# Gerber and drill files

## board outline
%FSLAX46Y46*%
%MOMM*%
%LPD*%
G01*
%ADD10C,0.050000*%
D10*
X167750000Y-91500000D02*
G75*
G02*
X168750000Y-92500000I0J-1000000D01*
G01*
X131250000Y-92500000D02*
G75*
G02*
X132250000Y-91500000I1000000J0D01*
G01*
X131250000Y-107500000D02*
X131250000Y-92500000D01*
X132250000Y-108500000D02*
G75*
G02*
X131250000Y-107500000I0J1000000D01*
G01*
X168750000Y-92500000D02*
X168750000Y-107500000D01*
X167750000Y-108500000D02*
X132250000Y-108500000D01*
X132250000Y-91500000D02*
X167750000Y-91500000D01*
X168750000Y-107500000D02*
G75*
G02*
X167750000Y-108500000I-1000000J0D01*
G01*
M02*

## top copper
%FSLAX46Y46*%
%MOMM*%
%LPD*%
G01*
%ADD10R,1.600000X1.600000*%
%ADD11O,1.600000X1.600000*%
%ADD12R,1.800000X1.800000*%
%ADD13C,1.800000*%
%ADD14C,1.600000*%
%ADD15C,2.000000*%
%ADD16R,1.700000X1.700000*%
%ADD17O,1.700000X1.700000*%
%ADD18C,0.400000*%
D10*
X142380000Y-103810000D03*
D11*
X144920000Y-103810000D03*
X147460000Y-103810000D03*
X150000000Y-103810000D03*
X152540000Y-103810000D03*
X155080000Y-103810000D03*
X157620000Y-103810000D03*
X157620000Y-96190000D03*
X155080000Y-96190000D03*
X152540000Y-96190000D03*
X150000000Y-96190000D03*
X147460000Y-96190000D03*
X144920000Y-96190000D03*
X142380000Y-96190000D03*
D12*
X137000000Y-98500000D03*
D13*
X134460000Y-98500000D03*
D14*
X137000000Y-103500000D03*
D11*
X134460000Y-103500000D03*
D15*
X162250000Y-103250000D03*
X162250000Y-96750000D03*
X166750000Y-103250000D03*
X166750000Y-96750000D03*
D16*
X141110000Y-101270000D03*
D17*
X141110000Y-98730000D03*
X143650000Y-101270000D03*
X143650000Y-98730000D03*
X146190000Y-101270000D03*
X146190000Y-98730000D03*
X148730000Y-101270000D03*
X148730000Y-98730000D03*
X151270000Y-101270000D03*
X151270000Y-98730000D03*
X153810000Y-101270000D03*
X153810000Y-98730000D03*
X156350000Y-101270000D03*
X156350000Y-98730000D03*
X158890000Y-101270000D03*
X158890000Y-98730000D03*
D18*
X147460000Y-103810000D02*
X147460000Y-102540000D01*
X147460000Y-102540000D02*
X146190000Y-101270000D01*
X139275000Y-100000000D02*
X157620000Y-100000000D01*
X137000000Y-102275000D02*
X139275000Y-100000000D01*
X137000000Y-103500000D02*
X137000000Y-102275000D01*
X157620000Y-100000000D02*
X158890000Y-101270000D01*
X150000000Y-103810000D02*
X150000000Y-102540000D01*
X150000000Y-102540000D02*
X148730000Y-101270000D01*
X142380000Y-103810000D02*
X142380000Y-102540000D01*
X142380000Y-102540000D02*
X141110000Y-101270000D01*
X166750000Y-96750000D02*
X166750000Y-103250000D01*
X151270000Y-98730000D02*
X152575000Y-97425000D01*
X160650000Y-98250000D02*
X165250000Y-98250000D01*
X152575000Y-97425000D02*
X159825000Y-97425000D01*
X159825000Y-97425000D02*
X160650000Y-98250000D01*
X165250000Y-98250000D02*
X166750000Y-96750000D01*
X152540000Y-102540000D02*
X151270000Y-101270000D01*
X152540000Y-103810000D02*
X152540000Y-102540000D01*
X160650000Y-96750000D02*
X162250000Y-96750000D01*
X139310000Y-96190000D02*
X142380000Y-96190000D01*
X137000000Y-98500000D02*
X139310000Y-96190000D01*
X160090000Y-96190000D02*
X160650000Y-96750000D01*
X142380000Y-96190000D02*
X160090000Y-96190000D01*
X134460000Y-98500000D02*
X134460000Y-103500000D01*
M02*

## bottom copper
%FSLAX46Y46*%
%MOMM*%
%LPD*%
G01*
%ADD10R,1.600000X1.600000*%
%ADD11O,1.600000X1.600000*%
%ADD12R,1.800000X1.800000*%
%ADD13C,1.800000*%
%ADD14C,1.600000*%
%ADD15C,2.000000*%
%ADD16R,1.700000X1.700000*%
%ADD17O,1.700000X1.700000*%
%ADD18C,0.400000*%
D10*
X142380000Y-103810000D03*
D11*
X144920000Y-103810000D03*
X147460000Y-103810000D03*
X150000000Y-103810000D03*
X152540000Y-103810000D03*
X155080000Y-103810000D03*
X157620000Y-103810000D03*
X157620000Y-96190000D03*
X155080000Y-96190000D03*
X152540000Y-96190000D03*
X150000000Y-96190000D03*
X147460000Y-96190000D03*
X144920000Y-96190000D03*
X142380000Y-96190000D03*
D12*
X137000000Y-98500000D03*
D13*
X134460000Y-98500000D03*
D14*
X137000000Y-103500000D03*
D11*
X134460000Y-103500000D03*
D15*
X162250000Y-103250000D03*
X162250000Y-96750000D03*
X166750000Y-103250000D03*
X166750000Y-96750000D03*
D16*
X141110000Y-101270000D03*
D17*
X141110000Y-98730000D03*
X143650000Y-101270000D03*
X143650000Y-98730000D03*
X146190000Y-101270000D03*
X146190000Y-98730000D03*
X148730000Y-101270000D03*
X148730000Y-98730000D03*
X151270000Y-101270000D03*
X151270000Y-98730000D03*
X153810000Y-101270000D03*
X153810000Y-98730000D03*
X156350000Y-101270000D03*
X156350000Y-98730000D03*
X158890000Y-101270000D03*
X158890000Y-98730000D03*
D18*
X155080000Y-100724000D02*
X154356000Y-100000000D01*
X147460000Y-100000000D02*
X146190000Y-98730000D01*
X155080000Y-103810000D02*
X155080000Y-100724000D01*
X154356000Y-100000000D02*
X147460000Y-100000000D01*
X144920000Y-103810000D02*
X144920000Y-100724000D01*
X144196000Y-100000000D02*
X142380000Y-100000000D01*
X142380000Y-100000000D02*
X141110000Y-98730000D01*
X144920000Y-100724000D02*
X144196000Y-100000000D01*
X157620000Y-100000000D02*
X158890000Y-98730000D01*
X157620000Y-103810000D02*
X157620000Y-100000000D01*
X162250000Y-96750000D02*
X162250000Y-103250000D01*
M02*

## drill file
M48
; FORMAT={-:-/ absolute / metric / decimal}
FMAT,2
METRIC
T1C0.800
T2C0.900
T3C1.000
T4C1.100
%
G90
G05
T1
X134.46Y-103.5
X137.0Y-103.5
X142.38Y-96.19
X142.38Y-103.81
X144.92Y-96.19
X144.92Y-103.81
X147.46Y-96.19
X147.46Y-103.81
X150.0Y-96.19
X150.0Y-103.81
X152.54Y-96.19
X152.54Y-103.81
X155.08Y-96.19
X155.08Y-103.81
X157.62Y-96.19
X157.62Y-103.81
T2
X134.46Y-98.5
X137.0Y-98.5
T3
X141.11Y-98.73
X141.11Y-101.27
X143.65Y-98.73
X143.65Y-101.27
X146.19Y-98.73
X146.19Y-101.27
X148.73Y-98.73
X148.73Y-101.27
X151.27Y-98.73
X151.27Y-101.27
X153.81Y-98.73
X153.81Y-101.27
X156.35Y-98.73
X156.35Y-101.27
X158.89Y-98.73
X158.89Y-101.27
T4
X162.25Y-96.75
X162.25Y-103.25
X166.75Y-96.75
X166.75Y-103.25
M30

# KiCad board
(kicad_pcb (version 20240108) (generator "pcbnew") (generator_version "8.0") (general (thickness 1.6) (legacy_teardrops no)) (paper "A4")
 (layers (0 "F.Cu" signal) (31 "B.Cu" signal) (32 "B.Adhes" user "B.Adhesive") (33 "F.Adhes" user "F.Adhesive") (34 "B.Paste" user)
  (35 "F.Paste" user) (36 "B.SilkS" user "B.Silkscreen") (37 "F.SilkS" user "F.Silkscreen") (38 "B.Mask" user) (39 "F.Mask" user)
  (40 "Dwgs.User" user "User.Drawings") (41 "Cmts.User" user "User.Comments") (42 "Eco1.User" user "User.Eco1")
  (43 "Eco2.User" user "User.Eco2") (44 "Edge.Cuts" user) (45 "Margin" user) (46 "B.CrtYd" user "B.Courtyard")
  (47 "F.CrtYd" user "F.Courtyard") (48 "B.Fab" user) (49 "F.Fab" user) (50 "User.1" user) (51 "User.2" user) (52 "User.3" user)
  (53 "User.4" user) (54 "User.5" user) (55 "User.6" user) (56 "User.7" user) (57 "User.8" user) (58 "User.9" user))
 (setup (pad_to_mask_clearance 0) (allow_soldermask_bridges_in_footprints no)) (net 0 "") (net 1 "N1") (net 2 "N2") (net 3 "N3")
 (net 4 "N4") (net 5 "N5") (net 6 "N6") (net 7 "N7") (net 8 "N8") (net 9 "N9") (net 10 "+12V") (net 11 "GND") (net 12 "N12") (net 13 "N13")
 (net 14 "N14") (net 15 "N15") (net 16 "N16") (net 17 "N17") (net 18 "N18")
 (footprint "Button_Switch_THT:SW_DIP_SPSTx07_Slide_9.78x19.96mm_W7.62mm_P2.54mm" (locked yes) (layer "F.Cu") (at 142.38 103.81 90)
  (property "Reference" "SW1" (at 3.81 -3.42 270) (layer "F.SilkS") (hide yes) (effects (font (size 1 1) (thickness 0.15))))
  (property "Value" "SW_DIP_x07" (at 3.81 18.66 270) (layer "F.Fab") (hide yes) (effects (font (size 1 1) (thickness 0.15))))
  (pad "1" thru_hole rect (at 0 0 90) (size 1.6 1.6) (drill 0.8) (layers "*.Cu" "*.Mask") (remove_unused_layers no) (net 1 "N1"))
  (pad "2" thru_hole oval (at 0 2.54 90) (size 1.6 1.6) (drill 0.8) (layers "*.Cu" "*.Mask") (remove_unused_layers no) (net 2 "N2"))
  (pad "3" thru_hole oval (at 0 5.08 90) (size 1.6 1.6) (drill 0.8) (layers "*.Cu" "*.Mask") (remove_unused_layers no) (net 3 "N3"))
  (pad "4" thru_hole oval (at 0 7.62 90) (size 1.6 1.6) (drill 0.8) (layers "*.Cu" "*.Mask") (remove_unused_layers no) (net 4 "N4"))
  (pad "5" thru_hole oval (at 0 10.16 90) (size 1.6 1.6) (drill 0.8) (layers "*.Cu" "*.Mask") (remove_unused_layers no) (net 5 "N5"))
  (pad "6" thru_hole oval (at 0 12.7 90) (size 1.6 1.6) (drill 0.8) (layers "*.Cu" "*.Mask") (remove_unused_layers no) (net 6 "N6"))
  (pad "7" thru_hole oval (at 0 15.24 90) (size 1.6 1.6) (drill 0.8) (layers "*.Cu" "*.Mask") (remove_unused_layers no) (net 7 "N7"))
  (pad "8" thru_hole oval (at 7.62 15.24 90) (size 1.6 1.6) (drill 0.8) (layers "*.Cu" "*.Mask") (remove_unused_layers no) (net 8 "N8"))
  (pad "9" thru_hole oval (at 7.62 12.7 90) (size 1.6 1.6) (drill 0.8) (layers "*.Cu" "*.Mask") (remove_unused_layers no) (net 8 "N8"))
  (pad "10" thru_hole oval (at 7.62 10.16 90) (size 1.6 1.6) (drill 0.8) (layers "*.Cu" "*.Mask") (remove_unused_layers no) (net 8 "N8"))
  (pad "11" thru_hole oval (at 7.62 7.62 90) (size 1.6 1.6) (drill 0.8) (layers "*.Cu" "*.Mask") (remove_unused_layers no) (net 8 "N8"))
  (pad "12" thru_hole oval (at 7.62 5.08 90) (size 1.6 1.6) (drill 0.8) (layers "*.Cu" "*.Mask") (remove_unused_layers no) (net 8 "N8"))
  (pad "13" thru_hole oval (at 7.62 2.54 90) (size 1.6 1.6) (drill 0.8) (layers "*.Cu" "*.Mask") (remove_unused_layers no) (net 8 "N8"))
  (pad "14" thru_hole oval (at 7.62 0 90) (size 1.6 1.6) (drill 0.8) (layers "*.Cu" "*.Mask") (remove_unused_layers no) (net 8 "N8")))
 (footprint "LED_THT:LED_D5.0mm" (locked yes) (layer "F.Cu") (at 137 98.5 180)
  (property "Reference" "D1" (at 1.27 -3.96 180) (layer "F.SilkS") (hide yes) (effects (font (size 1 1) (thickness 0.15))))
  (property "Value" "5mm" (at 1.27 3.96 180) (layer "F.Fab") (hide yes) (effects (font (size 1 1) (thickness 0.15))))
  (pad "1" thru_hole rect (at 0 0 180) (size 1.8 1.8) (drill 0.9) (layers "*.Cu" "*.Mask") (remove_unused_layers no) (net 8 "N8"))
  (pad "2" thru_hole circle (at 2.54 0 180) (size 1.8 1.8) (drill 0.9) (layers "*.Cu" "*.Mask") (remove_unused_layers no) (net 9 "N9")))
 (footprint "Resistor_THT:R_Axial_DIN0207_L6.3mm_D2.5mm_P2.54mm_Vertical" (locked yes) (layer "F.Cu") (at 137 103.5 180)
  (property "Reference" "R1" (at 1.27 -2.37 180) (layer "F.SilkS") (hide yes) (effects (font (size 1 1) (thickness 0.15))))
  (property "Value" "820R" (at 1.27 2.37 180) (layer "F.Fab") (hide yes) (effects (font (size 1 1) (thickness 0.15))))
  (pad "1" thru_hole circle (at 0 0 180) (size 1.6 1.6) (drill 0.8) (layers "*.Cu" "*.Mask") (remove_unused_layers no) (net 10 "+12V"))
  (pad "2" thru_hole oval (at 2.54 0 180) (size 1.6 1.6) (drill 0.8) (layers "*.Cu" "*.Mask") (remove_unused_layers no) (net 9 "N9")))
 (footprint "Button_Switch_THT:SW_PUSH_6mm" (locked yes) (layer "F.Cu") (at 162.25 103.25 90)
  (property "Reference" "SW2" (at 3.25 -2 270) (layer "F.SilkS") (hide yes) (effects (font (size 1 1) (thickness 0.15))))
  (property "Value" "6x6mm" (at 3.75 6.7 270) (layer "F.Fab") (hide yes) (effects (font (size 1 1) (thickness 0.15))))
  (pad "1" thru_hole circle (at 0 0 180) (size 2 2) (drill 1.1) (layers "*.Cu" "*.Mask") (remove_unused_layers no) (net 8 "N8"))
  (pad "1" thru_hole circle (at 6.5 0 180) (size 2 2) (drill 1.1) (layers "*.Cu" "*.Mask") (remove_unused_layers no) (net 8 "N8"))
  (pad "2" thru_hole circle (at 0 4.5 180) (size 2 2) (drill 1.1) (layers "*.Cu" "*.Mask") (remove_unused_layers no) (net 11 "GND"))
  (pad "2" thru_hole circle (at 6.5 4.5 180) (size 2 2) (drill 1.1) (layers "*.Cu" "*.Mask") (remove_unused_layers no) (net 11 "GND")))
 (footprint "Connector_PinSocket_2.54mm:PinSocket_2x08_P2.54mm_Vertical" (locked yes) (layer "B.Cu") (at 141.11 101.27 -90)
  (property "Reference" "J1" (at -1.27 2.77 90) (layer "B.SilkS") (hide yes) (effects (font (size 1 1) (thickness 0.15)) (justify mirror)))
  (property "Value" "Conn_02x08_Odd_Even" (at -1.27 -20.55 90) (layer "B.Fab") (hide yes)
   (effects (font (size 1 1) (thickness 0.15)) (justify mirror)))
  (pad "1" thru_hole rect (at 0 0 270) (size 1.7 1.7) (drill 1) (layers "*.Cu" "*.Mask") (remove_unused_layers no) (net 1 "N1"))
  (pad "2" thru_hole oval (at -2.54 0 270) (size 1.7 1.7) (drill 1) (layers "*.Cu" "*.Mask") (remove_unused_layers no) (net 2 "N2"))
  (pad "3" thru_hole oval (at 0 -2.54 270) (size 1.7 1.7) (drill 1) (layers "*.Cu" "*.Mask") (remove_unused_layers no) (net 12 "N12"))
  (pad "4" thru_hole oval (at -2.54 -2.54 270) (size 1.7 1.7) (drill 1) (layers "*.Cu" "*.Mask") (remove_unused_layers no) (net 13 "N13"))
  (pad "5" thru_hole oval (at 0 -5.08 270) (size 1.7 1.7) (drill 1) (layers "*.Cu" "*.Mask") (remove_unused_layers no) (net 3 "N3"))
  (pad "6" thru_hole oval (at -2.54 -5.08 270) (size 1.7 1.7) (drill 1) (layers "*.Cu" "*.Mask") (remove_unused_layers no) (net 6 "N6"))
  (pad "7" thru_hole oval (at 0 -7.62 270) (size 1.7 1.7) (drill 1) (layers "*.Cu" "*.Mask") (remove_unused_layers no) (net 4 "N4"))
  (pad "8" thru_hole oval (at -2.54 -7.62 270) (size 1.7 1.7) (drill 1) (layers "*.Cu" "*.Mask") (remove_unused_layers no) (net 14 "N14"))
  (pad "9" thru_hole oval (at 0 -10.16 270) (size 1.7 1.7) (drill 1) (layers "*.Cu" "*.Mask") (remove_unused_layers no) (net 5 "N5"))
  (pad "10" thru_hole oval (at -2.54 -10.16 270) (size 1.7 1.7) (drill 1) (layers "*.Cu" "*.Mask") (remove_unused_layers no) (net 11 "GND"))
  (pad "11" thru_hole oval (at 0 -12.7 270) (size 1.7 1.7) (drill 1) (layers "*.Cu" "*.Mask") (remove_unused_layers no) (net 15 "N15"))
  (pad "12" thru_hole oval (at -2.54 -12.7 270) (size 1.7 1.7) (drill 1) (layers "*.Cu" "*.Mask") (remove_unused_layers no) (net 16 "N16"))
  (pad "13" thru_hole oval (at 0 -15.24 270) (size 1.7 1.7) (drill 1) (layers "*.Cu" "*.Mask") (remove_unused_layers no) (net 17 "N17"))
  (pad "14" thru_hole oval (at -2.54 -15.24 270) (size 1.7 1.7) (drill 1) (layers "*.Cu" "*.Mask") (remove_unused_layers no) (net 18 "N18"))
  (pad "15" thru_hole oval (at 0 -17.78 270) (size 1.7 1.7) (drill 1) (layers "*.Cu" "*.Mask") (remove_unused_layers no) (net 10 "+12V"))
  (pad "16" thru_hole oval (at -2.54 -17.78 270) (size 1.7 1.7) (drill 1) (layers "*.Cu" "*.Mask") (remove_unused_layers no) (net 7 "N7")))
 (gr_arc (start 167.75 91.5) (mid 168.457107 91.792893) (end 168.75 92.5) (locked yes) (stroke (width 0.05) (type default))
  (layer "Edge.Cuts"))
 (gr_arc (start 131.25 92.5) (mid 131.542893 91.792893) (end 132.25 91.5) (locked yes) (stroke (width 0.05) (type default))
  (layer "Edge.Cuts"))
 (gr_line (start 131.25 107.5) (end 131.25 92.5) (locked yes) (stroke (width 0.05) (type default)) (layer "Edge.Cuts"))
 (gr_arc (start 132.25 108.5) (mid 131.542893 108.207107) (end 131.25 107.5) (locked yes) (stroke (width 0.05) (type default))
  (layer "Edge.Cuts"))
 (gr_line (start 168.75 92.5) (end 168.75 107.5) (locked yes) (stroke (width 0.05) (type default)) (layer "Edge.Cuts"))
 (gr_line (start 167.75 108.5) (end 132.25 108.5) (locked yes) (stroke (width 0.05) (type default)) (layer "Edge.Cuts"))
 (gr_line (start 132.25 91.5) (end 167.75 91.5) (locked yes) (stroke (width 0.05) (type default)) (layer "Edge.Cuts"))
 (gr_arc (start 168.75 107.5) (mid 168.457107 108.207107) (end 167.75 108.5) (locked yes) (stroke (width 0.05) (type default))
  (layer "Edge.Cuts"))
 (segment (start 147.46 103.81) (end 147.46 102.54) (width 0.4) (locked yes) (layer "F.Cu") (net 3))
 (segment (start 147.46 102.54) (end 146.19 101.27) (width 0.4) (locked yes) (layer "F.Cu") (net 3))
 (segment (start 139.275 100) (end 157.62 100) (width 0.4) (locked yes) (layer "F.Cu") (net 10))
 (segment (start 137 102.275) (end 139.275 100) (width 0.4) (locked yes) (layer "F.Cu") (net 10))
 (segment (start 137 103.5) (end 137 102.275) (width 0.4) (locked yes) (layer "F.Cu") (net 10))
 (segment (start 157.62 100) (end 158.89 101.27) (width 0.4) (locked yes) (layer "F.Cu") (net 10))
 (segment (start 150 103.81) (end 150 102.54) (width 0.4) (locked yes) (layer "F.Cu") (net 4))
 (segment (start 150 102.54) (end 148.73 101.27) (width 0.4) (locked yes) (layer "F.Cu") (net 4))
 (segment (start 142.38 103.81) (end 142.38 102.54) (width 0.4) (locked yes) (layer "F.Cu") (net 1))
 (segment (start 142.38 102.54) (end 141.11 101.27) (width 0.4) (locked yes) (layer "F.Cu") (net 1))
 (segment (start 155.08 100.724) (end 154.356 100) (width 0.4) (locked yes) (layer "B.Cu") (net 6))
 (segment (start 147.46 100) (end 146.19 98.73) (width 0.4) (locked yes) (layer "B.Cu") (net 6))
 (segment (start 155.08 103.81) (end 155.08 100.724) (width 0.4) (locked yes) (layer "B.Cu") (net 6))
 (segment (start 154.356 100) (end 147.46 100) (width 0.4) (locked yes) (layer "B.Cu") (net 6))
 (segment (start 144.92 103.81) (end 144.92 100.724) (width 0.4) (locked yes) (layer "B.Cu") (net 2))
 (segment (start 144.196 100) (end 142.38 100) (width 0.4) (locked yes) (layer "B.Cu") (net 2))
 (segment (start 142.38 100) (end 141.11 98.73) (width 0.4) (locked yes) (layer "B.Cu") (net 2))
 (segment (start 144.92 100.724) (end 144.196 100) (width 0.4) (locked yes) (layer "B.Cu") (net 2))
 (segment (start 166.75 96.75) (end 166.75 103.25) (width 0.4) (locked yes) (layer "F.Cu") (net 11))
 (segment (start 151.27 98.73) (end 152.575 97.425) (width 0.4) (locked yes) (layer "F.Cu") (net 11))
 (segment (start 160.65 98.25) (end 165.25 98.25) (width 0.4) (locked yes) (layer "F.Cu") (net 11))
 (segment (start 152.575 97.425) (end 159.825 97.425) (width 0.4) (locked yes) (layer "F.Cu") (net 11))
 (segment (start 159.825 97.425) (end 160.65 98.25) (width 0.4) (locked yes) (layer "F.Cu") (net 11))
 (segment (start 165.25 98.25) (end 166.75 96.75) (width 0.4) (locked yes) (layer "F.Cu") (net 11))
 (segment (start 157.62 100) (end 158.89 98.73) (width 0.4) (locked yes) (layer "B.Cu") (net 7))
 (segment (start 157.62 103.81) (end 157.62 100) (width 0.4) (locked yes) (layer "B.Cu") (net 7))
 (segment (start 152.54 102.54) (end 151.27 101.27) (width 0.4) (locked yes) (layer "F.Cu") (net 5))
 (segment (start 152.54 103.81) (end 152.54 102.54) (width 0.4) (locked yes) (layer "F.Cu") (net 5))
 (segment (start 160.65 96.75) (end 162.25 96.75) (width 0.4) (locked yes) (layer "F.Cu") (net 8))
 (segment (start 139.31 96.19) (end 142.38 96.19) (width 0.4) (locked yes) (layer "F.Cu") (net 8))
 (segment (start 137 98.5) (end 139.31 96.19) (width 0.4) (locked yes) (layer "F.Cu") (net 8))
 (segment (start 160.09 96.19) (end 160.65 96.75) (width 0.4) (locked yes) (layer "F.Cu") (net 8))
 (segment (start 142.38 96.19) (end 160.09 96.19) (width 0.4) (locked yes) (layer "F.Cu") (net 8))
 (segment (start 162.25 96.75) (end 162.25 103.25) (width 0.4) (locked yes) (layer "B.Cu") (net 8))
 (segment (start 134.46 98.5) (end 134.46 103.5) (width 0.4) (locked yes) (layer "F.Cu") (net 9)))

